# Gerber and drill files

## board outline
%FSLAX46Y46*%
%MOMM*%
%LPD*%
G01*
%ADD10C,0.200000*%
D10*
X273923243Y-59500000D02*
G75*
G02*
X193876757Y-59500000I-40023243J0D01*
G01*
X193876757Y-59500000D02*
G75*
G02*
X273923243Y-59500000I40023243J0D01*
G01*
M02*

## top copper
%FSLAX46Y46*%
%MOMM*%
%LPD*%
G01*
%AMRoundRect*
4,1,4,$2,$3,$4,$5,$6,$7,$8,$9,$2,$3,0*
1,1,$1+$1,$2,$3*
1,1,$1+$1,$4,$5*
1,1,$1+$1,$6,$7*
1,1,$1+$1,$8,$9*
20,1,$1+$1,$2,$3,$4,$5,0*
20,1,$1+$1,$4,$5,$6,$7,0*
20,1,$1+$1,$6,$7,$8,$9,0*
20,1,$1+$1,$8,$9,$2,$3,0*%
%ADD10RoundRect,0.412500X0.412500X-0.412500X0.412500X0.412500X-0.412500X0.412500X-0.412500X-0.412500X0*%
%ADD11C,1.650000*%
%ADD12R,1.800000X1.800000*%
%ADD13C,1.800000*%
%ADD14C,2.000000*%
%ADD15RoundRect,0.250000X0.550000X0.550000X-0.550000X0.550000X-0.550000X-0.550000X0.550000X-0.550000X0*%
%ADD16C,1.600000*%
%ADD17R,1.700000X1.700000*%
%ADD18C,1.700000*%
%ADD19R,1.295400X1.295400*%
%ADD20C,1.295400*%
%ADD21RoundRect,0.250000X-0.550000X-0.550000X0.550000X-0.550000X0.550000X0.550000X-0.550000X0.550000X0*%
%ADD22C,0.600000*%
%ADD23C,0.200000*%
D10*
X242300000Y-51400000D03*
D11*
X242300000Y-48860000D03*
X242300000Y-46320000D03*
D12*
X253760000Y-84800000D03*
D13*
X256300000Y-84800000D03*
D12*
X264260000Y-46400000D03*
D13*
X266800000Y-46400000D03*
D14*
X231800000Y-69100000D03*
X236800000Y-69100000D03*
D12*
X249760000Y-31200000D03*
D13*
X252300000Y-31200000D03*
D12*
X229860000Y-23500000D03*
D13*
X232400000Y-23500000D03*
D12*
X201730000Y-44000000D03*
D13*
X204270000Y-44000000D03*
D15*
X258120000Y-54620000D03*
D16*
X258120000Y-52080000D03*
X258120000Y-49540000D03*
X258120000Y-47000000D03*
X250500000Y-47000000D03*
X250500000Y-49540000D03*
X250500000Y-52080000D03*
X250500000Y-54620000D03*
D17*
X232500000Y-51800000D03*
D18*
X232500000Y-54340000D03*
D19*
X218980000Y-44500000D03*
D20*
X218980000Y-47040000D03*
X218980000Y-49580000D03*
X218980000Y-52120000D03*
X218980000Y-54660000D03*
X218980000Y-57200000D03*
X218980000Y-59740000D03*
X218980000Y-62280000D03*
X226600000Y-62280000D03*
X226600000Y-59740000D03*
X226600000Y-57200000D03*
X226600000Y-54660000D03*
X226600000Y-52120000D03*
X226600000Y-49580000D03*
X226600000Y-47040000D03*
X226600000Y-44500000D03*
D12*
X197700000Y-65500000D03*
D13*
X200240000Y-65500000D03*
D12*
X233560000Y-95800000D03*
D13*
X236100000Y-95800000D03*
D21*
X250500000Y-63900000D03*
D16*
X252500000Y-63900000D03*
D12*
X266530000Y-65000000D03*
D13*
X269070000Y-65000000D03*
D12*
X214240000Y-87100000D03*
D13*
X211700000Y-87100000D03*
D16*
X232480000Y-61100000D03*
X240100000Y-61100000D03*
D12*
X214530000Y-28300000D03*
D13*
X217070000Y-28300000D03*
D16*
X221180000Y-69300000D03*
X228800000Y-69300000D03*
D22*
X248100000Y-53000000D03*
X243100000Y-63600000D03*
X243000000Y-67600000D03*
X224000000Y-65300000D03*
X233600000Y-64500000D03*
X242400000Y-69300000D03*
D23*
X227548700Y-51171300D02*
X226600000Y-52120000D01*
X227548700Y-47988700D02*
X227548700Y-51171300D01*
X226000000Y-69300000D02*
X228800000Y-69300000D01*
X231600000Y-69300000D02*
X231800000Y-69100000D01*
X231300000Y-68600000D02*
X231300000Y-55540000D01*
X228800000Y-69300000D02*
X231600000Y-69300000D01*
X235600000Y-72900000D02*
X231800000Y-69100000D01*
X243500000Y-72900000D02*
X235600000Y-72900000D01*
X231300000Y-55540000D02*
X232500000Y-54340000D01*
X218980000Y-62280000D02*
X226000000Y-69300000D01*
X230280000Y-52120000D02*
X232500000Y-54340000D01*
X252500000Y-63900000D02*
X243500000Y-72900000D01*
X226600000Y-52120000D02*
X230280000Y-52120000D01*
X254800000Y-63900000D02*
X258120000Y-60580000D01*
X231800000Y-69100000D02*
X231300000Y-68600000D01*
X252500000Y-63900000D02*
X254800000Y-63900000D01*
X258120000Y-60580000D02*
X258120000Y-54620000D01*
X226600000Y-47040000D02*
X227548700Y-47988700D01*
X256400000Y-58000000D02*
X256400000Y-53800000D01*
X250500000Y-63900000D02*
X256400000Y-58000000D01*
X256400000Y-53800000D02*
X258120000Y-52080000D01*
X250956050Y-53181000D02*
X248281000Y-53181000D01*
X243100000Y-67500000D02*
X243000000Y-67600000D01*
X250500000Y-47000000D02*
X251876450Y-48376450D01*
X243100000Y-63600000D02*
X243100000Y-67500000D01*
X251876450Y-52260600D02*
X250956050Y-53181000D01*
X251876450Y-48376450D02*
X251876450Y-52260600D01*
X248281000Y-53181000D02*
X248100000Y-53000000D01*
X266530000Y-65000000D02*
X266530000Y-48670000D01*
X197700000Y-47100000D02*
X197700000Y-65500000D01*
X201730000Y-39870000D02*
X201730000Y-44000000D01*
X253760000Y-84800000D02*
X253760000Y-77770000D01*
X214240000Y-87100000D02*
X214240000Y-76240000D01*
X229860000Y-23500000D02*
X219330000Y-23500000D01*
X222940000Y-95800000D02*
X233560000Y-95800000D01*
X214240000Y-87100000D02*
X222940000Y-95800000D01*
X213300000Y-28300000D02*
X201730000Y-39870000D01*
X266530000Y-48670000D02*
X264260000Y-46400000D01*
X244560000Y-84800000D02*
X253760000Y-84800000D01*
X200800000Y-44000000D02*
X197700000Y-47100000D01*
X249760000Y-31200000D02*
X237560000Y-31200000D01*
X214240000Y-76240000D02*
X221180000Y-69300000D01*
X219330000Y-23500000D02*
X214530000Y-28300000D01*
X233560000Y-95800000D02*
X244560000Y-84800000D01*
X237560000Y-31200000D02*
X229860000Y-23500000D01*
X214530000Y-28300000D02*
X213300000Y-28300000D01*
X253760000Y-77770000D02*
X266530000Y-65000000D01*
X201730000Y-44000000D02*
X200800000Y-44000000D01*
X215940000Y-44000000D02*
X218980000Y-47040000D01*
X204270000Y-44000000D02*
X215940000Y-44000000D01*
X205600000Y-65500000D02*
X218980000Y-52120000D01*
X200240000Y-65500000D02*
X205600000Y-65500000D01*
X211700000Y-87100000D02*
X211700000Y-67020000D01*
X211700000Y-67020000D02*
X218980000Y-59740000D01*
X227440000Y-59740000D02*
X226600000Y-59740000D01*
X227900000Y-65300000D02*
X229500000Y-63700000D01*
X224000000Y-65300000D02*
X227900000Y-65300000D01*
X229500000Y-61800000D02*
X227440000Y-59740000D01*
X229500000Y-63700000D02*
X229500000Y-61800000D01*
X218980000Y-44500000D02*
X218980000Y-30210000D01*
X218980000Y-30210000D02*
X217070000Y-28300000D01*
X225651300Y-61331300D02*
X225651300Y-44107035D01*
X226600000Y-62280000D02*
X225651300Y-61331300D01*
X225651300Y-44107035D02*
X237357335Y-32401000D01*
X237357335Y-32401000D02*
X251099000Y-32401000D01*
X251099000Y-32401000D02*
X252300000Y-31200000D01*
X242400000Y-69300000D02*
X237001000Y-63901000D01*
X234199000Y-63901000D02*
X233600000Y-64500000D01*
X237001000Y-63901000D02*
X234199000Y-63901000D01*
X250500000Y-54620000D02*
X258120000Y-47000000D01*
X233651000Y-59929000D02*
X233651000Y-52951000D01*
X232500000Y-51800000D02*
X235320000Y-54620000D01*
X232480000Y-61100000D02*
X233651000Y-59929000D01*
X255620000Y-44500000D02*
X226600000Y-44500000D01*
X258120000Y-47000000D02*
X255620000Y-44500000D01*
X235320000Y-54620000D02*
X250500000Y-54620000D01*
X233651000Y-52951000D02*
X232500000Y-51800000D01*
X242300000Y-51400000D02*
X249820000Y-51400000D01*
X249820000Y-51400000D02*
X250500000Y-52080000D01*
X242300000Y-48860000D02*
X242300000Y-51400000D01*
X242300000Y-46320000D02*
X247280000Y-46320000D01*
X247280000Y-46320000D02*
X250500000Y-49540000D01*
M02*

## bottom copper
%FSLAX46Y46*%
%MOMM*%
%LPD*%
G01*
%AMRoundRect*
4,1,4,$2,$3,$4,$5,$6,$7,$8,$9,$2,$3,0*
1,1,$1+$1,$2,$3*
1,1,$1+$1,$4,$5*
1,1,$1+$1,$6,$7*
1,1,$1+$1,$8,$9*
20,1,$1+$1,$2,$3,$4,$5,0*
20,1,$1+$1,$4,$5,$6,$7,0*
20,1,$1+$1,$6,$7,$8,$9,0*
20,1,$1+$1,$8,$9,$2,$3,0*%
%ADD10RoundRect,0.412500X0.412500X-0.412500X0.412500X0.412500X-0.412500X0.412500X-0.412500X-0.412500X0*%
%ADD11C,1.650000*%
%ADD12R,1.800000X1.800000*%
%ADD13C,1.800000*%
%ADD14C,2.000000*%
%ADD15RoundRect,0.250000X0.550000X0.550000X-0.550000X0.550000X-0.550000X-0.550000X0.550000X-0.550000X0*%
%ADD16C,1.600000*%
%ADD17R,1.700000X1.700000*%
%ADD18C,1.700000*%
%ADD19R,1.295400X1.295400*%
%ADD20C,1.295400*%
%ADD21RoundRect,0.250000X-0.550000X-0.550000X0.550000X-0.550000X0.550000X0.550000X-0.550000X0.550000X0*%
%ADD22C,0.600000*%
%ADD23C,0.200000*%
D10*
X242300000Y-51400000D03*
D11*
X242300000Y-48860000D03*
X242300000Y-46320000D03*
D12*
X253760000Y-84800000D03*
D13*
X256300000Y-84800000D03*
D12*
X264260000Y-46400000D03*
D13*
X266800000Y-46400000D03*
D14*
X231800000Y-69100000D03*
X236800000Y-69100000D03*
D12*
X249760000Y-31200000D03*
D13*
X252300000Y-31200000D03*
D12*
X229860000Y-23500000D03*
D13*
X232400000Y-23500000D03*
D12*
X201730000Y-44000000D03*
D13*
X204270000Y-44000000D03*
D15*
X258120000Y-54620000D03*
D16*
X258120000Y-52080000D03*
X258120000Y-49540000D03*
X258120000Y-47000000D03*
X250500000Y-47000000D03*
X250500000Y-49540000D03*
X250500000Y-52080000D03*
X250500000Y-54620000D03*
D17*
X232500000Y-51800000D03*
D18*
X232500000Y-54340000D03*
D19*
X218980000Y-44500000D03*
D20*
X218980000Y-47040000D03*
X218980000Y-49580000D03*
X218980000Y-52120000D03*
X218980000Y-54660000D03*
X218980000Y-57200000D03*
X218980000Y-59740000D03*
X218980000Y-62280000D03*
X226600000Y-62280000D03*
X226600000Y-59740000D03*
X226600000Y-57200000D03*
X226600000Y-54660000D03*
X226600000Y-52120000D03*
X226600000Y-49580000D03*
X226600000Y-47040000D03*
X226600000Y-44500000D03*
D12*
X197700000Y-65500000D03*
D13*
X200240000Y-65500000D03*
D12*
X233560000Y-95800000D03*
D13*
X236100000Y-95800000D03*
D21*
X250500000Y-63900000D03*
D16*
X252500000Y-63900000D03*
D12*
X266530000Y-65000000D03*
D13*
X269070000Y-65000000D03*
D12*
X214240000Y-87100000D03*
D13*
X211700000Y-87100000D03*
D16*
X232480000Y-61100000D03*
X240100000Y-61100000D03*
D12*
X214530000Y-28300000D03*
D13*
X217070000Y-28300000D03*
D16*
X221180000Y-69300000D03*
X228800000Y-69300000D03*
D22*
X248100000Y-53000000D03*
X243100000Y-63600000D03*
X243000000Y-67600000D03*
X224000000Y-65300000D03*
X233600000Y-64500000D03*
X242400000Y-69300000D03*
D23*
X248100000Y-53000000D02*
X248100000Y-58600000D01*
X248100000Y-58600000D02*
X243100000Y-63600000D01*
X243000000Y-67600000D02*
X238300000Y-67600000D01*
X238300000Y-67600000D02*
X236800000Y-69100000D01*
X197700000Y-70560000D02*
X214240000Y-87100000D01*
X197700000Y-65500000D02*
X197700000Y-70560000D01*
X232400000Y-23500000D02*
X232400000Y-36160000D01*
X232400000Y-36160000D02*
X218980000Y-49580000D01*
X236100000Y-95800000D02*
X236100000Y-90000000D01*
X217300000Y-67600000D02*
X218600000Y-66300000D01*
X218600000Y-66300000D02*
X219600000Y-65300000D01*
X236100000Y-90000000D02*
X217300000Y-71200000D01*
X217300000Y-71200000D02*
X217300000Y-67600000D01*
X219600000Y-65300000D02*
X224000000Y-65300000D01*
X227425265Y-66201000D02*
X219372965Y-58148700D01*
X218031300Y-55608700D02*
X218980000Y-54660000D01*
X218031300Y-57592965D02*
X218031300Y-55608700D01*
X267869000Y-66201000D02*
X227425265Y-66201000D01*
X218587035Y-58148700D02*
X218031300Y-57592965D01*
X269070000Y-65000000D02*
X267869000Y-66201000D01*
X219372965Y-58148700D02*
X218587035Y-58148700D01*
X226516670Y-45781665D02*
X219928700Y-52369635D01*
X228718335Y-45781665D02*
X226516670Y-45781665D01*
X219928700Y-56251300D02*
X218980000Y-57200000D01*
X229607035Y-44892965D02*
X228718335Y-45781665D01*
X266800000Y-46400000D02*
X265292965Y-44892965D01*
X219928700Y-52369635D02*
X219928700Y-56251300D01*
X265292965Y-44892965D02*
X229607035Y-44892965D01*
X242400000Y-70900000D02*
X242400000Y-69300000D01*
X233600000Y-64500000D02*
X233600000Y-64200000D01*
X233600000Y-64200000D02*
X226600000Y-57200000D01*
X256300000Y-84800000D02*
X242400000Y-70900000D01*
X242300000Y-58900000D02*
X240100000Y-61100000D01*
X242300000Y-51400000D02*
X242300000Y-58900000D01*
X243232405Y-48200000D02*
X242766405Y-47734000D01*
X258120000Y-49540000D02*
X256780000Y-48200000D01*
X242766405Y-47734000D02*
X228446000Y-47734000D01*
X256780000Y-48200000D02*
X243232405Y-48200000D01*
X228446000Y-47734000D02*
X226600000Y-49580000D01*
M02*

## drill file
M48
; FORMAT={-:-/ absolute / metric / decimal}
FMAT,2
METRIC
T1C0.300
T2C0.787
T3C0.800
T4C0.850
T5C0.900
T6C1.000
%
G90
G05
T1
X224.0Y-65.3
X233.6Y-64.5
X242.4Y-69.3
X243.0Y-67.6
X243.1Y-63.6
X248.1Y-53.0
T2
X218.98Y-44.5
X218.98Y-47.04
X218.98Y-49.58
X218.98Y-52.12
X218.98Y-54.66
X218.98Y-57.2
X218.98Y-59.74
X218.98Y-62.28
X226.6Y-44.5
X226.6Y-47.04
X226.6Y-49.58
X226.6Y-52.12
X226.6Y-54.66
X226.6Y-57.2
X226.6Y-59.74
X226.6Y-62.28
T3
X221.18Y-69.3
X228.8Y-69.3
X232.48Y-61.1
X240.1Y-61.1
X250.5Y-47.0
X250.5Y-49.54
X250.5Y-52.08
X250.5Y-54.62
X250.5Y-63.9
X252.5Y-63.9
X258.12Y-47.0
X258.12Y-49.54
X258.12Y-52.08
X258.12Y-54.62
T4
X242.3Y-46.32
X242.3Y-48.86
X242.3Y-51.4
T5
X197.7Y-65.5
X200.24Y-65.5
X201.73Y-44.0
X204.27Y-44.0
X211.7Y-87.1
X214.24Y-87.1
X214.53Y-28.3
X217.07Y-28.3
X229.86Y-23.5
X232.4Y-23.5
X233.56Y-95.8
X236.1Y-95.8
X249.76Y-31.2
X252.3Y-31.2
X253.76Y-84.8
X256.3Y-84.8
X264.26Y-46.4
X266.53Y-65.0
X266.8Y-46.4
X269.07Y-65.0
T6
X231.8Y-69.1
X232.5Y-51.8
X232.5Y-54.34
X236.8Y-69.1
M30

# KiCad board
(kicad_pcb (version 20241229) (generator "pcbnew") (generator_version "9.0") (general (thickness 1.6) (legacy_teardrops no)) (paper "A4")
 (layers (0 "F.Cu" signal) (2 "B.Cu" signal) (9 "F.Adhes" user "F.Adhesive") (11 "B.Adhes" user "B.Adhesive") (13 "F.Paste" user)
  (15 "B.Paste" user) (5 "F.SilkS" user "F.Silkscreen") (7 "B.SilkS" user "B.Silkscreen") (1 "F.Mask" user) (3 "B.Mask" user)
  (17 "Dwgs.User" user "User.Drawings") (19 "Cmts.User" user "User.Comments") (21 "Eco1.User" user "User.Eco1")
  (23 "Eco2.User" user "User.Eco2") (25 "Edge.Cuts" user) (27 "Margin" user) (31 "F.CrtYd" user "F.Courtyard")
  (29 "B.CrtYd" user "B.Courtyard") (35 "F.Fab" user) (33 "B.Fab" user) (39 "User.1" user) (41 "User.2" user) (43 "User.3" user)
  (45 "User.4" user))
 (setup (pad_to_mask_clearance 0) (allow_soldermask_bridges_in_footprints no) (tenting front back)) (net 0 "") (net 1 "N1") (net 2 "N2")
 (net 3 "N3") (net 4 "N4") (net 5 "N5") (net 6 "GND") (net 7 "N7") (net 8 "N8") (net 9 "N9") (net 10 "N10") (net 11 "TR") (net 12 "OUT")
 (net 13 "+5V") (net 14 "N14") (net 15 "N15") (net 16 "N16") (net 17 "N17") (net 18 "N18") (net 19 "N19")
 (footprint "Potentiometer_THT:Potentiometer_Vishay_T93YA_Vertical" (layer "F.Cu") (at 242.3 51.4 90)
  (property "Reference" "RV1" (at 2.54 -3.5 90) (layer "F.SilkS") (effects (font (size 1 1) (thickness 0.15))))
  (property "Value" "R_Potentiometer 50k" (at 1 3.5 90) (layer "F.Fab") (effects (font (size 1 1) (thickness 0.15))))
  (pad "1" thru_hole roundrect (at 0 0 90) (size 1.65 1.65) (drill 0.85) (layers "*.Cu" "*.Mask") (remove_unused_layers no)
   (roundrect_rratio 0.25) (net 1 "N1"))
  (pad "2" thru_hole circle (at 2.54 0 90) (size 1.65 1.65) (drill 0.85) (layers "*.Cu" "*.Mask") (remove_unused_layers no) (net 1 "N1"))
  (pad "3" thru_hole circle (at 5.08 0 90) (size 1.65 1.65) (drill 0.85) (layers "*.Cu" "*.Mask") (remove_unused_layers no) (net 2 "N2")))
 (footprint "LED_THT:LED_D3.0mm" (layer "F.Cu") (at 253.76 84.8)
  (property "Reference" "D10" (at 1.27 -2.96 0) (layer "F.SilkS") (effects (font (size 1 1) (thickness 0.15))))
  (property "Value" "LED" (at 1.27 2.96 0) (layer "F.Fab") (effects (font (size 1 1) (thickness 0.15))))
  (pad "1" thru_hole rect (at 0 0) (size 1.8 1.8) (drill 0.9) (layers "*.Cu" "*.Mask") (remove_unused_layers no) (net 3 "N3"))
  (pad "2" thru_hole circle (at 2.54 0) (size 1.8 1.8) (drill 0.9) (layers "*.Cu" "*.Mask") (remove_unused_layers no) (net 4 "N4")))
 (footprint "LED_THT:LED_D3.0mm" (layer "F.Cu") (at 264.26 46.4)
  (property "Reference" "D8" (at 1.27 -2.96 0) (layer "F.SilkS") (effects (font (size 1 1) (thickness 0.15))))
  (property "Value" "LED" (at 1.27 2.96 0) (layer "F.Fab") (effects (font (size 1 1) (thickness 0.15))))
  (pad "1" thru_hole rect (at 0 0) (size 1.8 1.8) (drill 0.9) (layers "*.Cu" "*.Mask") (remove_unused_layers no) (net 3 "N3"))
  (pad "2" thru_hole circle (at 2.54 0) (size 1.8 1.8) (drill 0.9) (layers "*.Cu" "*.Mask") (remove_unused_layers no) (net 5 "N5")))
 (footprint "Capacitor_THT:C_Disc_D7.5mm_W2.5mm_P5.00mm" (layer "F.Cu") (at 231.8 69.1)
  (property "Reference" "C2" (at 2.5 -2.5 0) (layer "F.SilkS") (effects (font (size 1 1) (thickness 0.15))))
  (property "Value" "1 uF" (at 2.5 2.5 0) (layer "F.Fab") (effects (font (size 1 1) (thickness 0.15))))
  (pad "1" thru_hole circle (at 0 0) (size 2 2) (drill 1) (layers "*.Cu" "*.Mask") (remove_unused_layers no) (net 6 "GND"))
  (pad "2" thru_hole circle (at 5 0) (size 2 2) (drill 1) (layers "*.Cu" "*.Mask") (remove_unused_layers no) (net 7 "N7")))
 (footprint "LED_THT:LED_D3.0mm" (layer "F.Cu") (at 249.76 31.2)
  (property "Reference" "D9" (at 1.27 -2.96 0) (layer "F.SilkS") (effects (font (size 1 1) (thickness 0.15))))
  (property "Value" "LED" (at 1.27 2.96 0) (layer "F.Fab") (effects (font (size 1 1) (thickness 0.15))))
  (pad "1" thru_hole rect (at 0 0) (size 1.8 1.8) (drill 0.9) (layers "*.Cu" "*.Mask") (remove_unused_layers no) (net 3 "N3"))
  (pad "2" thru_hole circle (at 2.54 0) (size 1.8 1.8) (drill 0.9) (layers "*.Cu" "*.Mask") (remove_unused_layers no) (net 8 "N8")))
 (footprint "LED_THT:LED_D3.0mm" (layer "F.Cu") (at 229.86 23.5)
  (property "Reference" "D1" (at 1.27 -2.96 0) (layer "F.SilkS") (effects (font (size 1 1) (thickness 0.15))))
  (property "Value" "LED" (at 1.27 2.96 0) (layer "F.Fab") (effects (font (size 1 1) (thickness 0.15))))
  (pad "1" thru_hole rect (at 0 0) (size 1.8 1.8) (drill 0.9) (layers "*.Cu" "*.Mask") (remove_unused_layers no) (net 3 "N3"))
  (pad "2" thru_hole circle (at 2.54 0) (size 1.8 1.8) (drill 0.9) (layers "*.Cu" "*.Mask") (remove_unused_layers no) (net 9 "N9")))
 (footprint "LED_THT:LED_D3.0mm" (layer "F.Cu") (at 201.73 44)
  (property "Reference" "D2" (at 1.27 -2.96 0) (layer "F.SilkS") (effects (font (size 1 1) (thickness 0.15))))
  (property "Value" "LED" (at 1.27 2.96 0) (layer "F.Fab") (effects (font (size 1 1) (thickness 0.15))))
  (pad "1" thru_hole rect (at 0 0) (size 1.8 1.8) (drill 0.9) (layers "*.Cu" "*.Mask") (remove_unused_layers no) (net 3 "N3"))
  (pad "2" thru_hole circle (at 2.54 0) (size 1.8 1.8) (drill 0.9) (layers "*.Cu" "*.Mask") (remove_unused_layers no) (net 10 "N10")))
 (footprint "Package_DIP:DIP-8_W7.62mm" (layer "F.Cu") (at 258.12 54.62 180)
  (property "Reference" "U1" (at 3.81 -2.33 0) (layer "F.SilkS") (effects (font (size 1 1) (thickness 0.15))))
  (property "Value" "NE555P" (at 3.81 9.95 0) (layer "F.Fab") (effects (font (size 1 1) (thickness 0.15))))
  (pad "1" thru_hole roundrect (at 0 0 180) (size 1.6 1.6) (drill 0.8) (layers "*.Cu" "*.Mask") (remove_unused_layers no)
   (roundrect_rratio 0.15625) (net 6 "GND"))
  (pad "2" thru_hole circle (at 0 2.54 180) (size 1.6 1.6) (drill 0.8) (layers "*.Cu" "*.Mask") (remove_unused_layers no) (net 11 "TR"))
  (pad "3" thru_hole circle (at 0 5.08 180) (size 1.6 1.6) (drill 0.8) (layers "*.Cu" "*.Mask") (remove_unused_layers no) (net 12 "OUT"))
  (pad "4" thru_hole circle (at 0 7.62 180) (size 1.6 1.6) (drill 0.8) (layers "*.Cu" "*.Mask") (remove_unused_layers no) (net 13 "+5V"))
  (pad "5" thru_hole circle (at 7.62 7.62 180) (size 1.6 1.6) (drill 0.8) (layers "*.Cu" "*.Mask") (remove_unused_layers no) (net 7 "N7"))
  (pad "6" thru_hole circle (at 7.62 5.08 180) (size 1.6 1.6) (drill 0.8) (layers "*.Cu" "*.Mask") (remove_unused_layers no) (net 2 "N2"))
  (pad "7" thru_hole circle (at 7.62 2.54 180) (size 1.6 1.6) (drill 0.8) (layers "*.Cu" "*.Mask") (remove_unused_layers no) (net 1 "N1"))
  (pad "8" thru_hole circle (at 7.62 0 180) (size 1.6 1.6) (drill 0.8) (layers "*.Cu" "*.Mask") (remove_unused_layers no) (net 13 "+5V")))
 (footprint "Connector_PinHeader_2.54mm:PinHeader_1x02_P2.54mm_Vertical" (layer "F.Cu") (at 232.5 51.8)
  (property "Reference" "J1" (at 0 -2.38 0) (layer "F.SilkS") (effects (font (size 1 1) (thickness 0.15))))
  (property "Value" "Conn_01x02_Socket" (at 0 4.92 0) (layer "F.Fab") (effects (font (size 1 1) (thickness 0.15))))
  (pad "1" thru_hole rect (at 0 0) (size 1.7 1.7) (drill 1) (layers "*.Cu" "*.Mask") (remove_unused_layers no) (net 13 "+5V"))
  (pad "2" thru_hole circle (at 0 2.54) (size 1.7 1.7) (drill 1) (layers "*.Cu" "*.Mask") (remove_unused_layers no) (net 6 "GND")))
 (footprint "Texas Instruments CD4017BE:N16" (layer "F.Cu") (at 226.6 62.28)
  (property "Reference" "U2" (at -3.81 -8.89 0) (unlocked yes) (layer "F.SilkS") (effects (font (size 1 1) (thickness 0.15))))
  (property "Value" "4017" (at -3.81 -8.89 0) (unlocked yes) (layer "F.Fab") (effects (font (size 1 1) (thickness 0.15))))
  (pad "1" thru_hole rect (at -7.62 -17.78) (size 1.2954 1.2954) (drill 0.7874) (layers "*.Cu" "*.Mask") (remove_unused_layers no)
   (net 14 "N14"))
  (pad "2" thru_hole circle (at -7.62 -15.24) (size 1.2954 1.2954) (drill 0.7874) (layers "*.Cu" "*.Mask") (remove_unused_layers no)
   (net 10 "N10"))
  (pad "3" thru_hole circle (at -7.62 -12.7) (size 1.2954 1.2954) (drill 0.7874) (layers "*.Cu" "*.Mask") (remove_unused_layers no)
   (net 9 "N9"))
  (pad "4" thru_hole circle (at -7.62 -10.16) (size 1.2954 1.2954) (drill 0.7874) (layers "*.Cu" "*.Mask") (remove_unused_layers no)
   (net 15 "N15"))
  (pad "5" thru_hole circle (at -7.62 -7.62) (size 1.2954 1.2954) (drill 0.7874) (layers "*.Cu" "*.Mask") (remove_unused_layers no)
   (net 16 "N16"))
  (pad "6" thru_hole circle (at -7.62 -5.08) (size 1.2954 1.2954) (drill 0.7874) (layers "*.Cu" "*.Mask") (remove_unused_layers no)
   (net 5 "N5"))
  (pad "7" thru_hole circle (at -7.62 -2.54) (size 1.2954 1.2954) (drill 0.7874) (layers "*.Cu" "*.Mask") (remove_unused_layers no)
   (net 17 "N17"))
  (pad "8" thru_hole circle (at -7.62 0) (size 1.2954 1.2954) (drill 0.7874) (layers "*.Cu" "*.Mask") (remove_unused_layers no)
   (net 6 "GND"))
  (pad "9" thru_hole circle (at 0 0) (size 1.2954 1.2954) (drill 0.7874) (layers "*.Cu" "*.Mask") (remove_unused_layers no) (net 8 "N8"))
  (pad "10" thru_hole circle (at 0 -2.54) (size 1.2954 1.2954) (drill 0.7874) (layers "*.Cu" "*.Mask") (remove_unused_layers no)
   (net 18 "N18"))
  (pad "11" thru_hole circle (at 0 -5.08) (size 1.2954 1.2954) (drill 0.7874) (layers "*.Cu" "*.Mask") (remove_unused_layers no)
   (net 4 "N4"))
  (pad "12" thru_hole circle (at 0 -7.62) (size 1.2954 1.2954) (drill 0.7874) (layers "*.Cu" "*.Mask") (remove_unused_layers no)
   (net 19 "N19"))
  (pad "13" thru_hole circle (at 0 -10.16) (size 1.2954 1.2954) (drill 0.7874) (layers "*.Cu" "*.Mask") (remove_unused_layers no)
   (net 6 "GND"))
  (pad "14" thru_hole circle (at 0 -12.7) (size 1.2954 1.2954) (drill 0.7874) (layers "*.Cu" "*.Mask") (remove_unused_layers no)
   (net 12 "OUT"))
  (pad "15" thru_hole circle (at 0 -15.24) (size 1.2954 1.2954) (drill 0.7874) (layers "*.Cu" "*.Mask") (remove_unused_layers no)
   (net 6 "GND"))
  (pad "16" thru_hole circle (at 0 -17.78) (size 1.2954 1.2954) (drill 0.7874) (layers "*.Cu" "*.Mask") (remove_unused_layers no)
   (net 13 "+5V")))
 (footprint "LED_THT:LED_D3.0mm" (layer "F.Cu") (at 197.7 65.5)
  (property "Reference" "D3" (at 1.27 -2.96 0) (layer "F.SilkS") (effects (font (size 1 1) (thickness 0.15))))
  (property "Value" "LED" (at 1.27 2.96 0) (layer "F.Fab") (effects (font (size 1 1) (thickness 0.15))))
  (pad "1" thru_hole rect (at 0 0) (size 1.8 1.8) (drill 0.9) (layers "*.Cu" "*.Mask") (remove_unused_layers no) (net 3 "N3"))
  (pad "2" thru_hole circle (at 2.54 0) (size 1.8 1.8) (drill 0.9) (layers "*.Cu" "*.Mask") (remove_unused_layers no) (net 15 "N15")))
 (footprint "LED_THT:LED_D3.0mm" (layer "F.Cu") (at 233.56 95.8)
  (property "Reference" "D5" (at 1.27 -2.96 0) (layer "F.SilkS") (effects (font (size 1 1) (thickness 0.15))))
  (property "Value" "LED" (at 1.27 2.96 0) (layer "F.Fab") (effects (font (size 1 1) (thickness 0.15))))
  (pad "1" thru_hole rect (at 0 0) (size 1.8 1.8) (drill 0.9) (layers "*.Cu" "*.Mask") (remove_unused_layers no) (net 3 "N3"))
  (pad "2" thru_hole circle (at 2.54 0) (size 1.8 1.8) (drill 0.9) (layers "*.Cu" "*.Mask") (remove_unused_layers no) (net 18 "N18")))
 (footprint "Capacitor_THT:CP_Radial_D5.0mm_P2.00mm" (layer "F.Cu") (at 250.5 63.9)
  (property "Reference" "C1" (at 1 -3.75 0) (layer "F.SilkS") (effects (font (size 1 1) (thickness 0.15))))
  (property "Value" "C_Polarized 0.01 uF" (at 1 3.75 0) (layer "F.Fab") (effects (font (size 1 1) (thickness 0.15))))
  (pad "1" thru_hole roundrect (at 0 0) (size 1.6 1.6) (drill 0.8) (layers "*.Cu" "*.Mask") (remove_unused_layers no)
   (roundrect_rratio 0.15625) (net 11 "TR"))
  (pad "2" thru_hole circle (at 2 0) (size 1.6 1.6) (drill 0.8) (layers "*.Cu" "*.Mask") (remove_unused_layers no) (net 6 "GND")))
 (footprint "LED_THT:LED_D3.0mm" (layer "F.Cu") (at 266.53 65)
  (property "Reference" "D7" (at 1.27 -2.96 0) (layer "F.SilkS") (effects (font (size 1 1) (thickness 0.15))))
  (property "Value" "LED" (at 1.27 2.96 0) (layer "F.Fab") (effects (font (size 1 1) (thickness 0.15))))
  (pad "1" thru_hole rect (at 0 0) (size 1.8 1.8) (drill 0.9) (layers "*.Cu" "*.Mask") (remove_unused_layers no) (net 3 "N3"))
  (pad "2" thru_hole circle (at 2.54 0) (size 1.8 1.8) (drill 0.9) (layers "*.Cu" "*.Mask") (remove_unused_layers no) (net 16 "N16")))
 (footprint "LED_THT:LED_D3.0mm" (layer "F.Cu") (at 214.24 87.1 180)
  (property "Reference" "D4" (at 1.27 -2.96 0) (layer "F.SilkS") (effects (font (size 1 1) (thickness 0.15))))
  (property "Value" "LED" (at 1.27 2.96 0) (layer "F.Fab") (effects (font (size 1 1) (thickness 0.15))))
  (pad "1" thru_hole rect (at 0 0 180) (size 1.8 1.8) (drill 0.9) (layers "*.Cu" "*.Mask") (remove_unused_layers no) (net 3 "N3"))
  (pad "2" thru_hole circle (at 2.54 0 180) (size 1.8 1.8) (drill 0.9) (layers "*.Cu" "*.Mask") (remove_unused_layers no) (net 17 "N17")))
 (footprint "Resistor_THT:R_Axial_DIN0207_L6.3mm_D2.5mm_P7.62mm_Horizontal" (layer "F.Cu") (at 232.48 61.1)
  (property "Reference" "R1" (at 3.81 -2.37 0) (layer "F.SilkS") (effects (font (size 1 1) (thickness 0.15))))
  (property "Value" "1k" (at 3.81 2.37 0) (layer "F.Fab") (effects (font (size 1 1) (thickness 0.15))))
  (pad "1" thru_hole circle (at 0 0) (size 1.6 1.6) (drill 0.8) (layers "*.Cu" "*.Mask") (remove_unused_layers no) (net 13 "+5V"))
  (pad "2" thru_hole circle (at 7.62 0) (size 1.6 1.6) (drill 0.8) (layers "*.Cu" "*.Mask") (remove_unused_layers no) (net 1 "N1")))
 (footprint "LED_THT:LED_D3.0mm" (layer "F.Cu") (at 214.53 28.3)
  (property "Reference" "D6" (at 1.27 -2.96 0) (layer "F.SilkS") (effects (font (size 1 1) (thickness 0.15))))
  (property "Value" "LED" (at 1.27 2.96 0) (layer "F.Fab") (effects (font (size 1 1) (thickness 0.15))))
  (pad "1" thru_hole rect (at 0 0) (size 1.8 1.8) (drill 0.9) (layers "*.Cu" "*.Mask") (remove_unused_layers no) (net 3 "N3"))
  (pad "2" thru_hole circle (at 2.54 0) (size 1.8 1.8) (drill 0.9) (layers "*.Cu" "*.Mask") (remove_unused_layers no) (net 14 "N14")))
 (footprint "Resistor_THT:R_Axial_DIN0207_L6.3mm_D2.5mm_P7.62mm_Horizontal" (layer "F.Cu") (at 221.18 69.3)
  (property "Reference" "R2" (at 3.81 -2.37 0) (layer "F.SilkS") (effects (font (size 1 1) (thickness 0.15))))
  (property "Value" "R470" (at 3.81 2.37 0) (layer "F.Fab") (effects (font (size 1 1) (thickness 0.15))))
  (pad "1" thru_hole circle (at 0 0) (size 1.6 1.6) (drill 0.8) (layers "*.Cu" "*.Mask") (remove_unused_layers no) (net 3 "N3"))
  (pad "2" thru_hole circle (at 7.62 0) (size 1.6 1.6) (drill 0.8) (layers "*.Cu" "*.Mask") (remove_unused_layers no) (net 6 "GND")))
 (gr_circle (center 233.9 59.5) (end 267 82) (stroke (width 0.2) (type solid)) (fill no) (layer "Edge.Cuts"))
 (segment (start 227.5487 51.1713) (end 226.6 52.12) (width 0.2) (layer "F.Cu") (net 6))
 (segment (start 227.5487 47.9887) (end 227.5487 51.1713) (width 0.2) (layer "F.Cu") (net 6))
 (segment (start 226 69.3) (end 228.8 69.3) (width 0.2) (layer "F.Cu") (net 6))
 (segment (start 231.6 69.3) (end 231.8 69.1) (width 0.2) (layer "F.Cu") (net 6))
 (segment (start 231.3 68.6) (end 231.3 55.54) (width 0.2) (layer "F.Cu") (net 6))
 (segment (start 228.8 69.3) (end 231.6 69.3) (width 0.2) (layer "F.Cu") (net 6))
 (segment (start 235.6 72.9) (end 231.8 69.1) (width 0.2) (layer "F.Cu") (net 6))
 (segment (start 243.5 72.9) (end 235.6 72.9) (width 0.2) (layer "F.Cu") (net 6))
 (segment (start 231.3 55.54) (end 232.5 54.34) (width 0.2) (layer "F.Cu") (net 6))
 (segment (start 218.98 62.28) (end 226 69.3) (width 0.2) (layer "F.Cu") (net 6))
 (segment (start 230.28 52.12) (end 232.5 54.34) (width 0.2) (layer "F.Cu") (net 6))
 (segment (start 252.5 63.9) (end 243.5 72.9) (width 0.2) (layer "F.Cu") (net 6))
 (segment (start 226.6 52.12) (end 230.28 52.12) (width 0.2) (layer "F.Cu") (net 6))
 (segment (start 254.8 63.9) (end 258.12 60.58) (width 0.2) (layer "F.Cu") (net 6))
 (segment (start 231.8 69.1) (end 231.3 68.6) (width 0.2) (layer "F.Cu") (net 6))
 (segment (start 252.5 63.9) (end 254.8 63.9) (width 0.2) (layer "F.Cu") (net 6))
 (segment (start 258.12 60.58) (end 258.12 54.62) (width 0.2) (layer "F.Cu") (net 6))
 (segment (start 226.6 47.04) (end 227.5487 47.9887) (width 0.2) (layer "F.Cu") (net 6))
 (segment (start 256.4 58) (end 256.4 53.8) (width 0.2) (layer "F.Cu") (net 11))
 (segment (start 250.5 63.9) (end 256.4 58) (width 0.2) (layer "F.Cu") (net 11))
 (segment (start 256.4 53.8) (end 258.12 52.08) (width 0.2) (layer "F.Cu") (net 11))
 (segment (start 250.95605 53.181) (end 248.281 53.181) (width 0.2) (layer "F.Cu") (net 7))
 (segment (start 243.1 67.5) (end 243 67.6) (width 0.2) (layer "F.Cu") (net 7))
 (segment (start 250.5 47) (end 251.87645 48.37645) (width 0.2) (layer "F.Cu") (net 7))
 (segment (start 243.1 63.6) (end 243.1 67.5) (width 0.2) (layer "F.Cu") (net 7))
 (segment (start 251.87645 52.2606) (end 250.95605 53.181) (width 0.2) (layer "F.Cu") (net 7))
 (segment (start 251.87645 48.37645) (end 251.87645 52.2606) (width 0.2) (layer "F.Cu") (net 7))
 (segment (start 248.281 53.181) (end 248.1 53) (width 0.2) (layer "F.Cu") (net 7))
 (via (at 248.1 53) (size 0.6) (drill 0.3) (layers "F.Cu" "B.Cu") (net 7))
 (via (at 243.1 63.6) (size 0.6) (drill 0.3) (layers "F.Cu" "B.Cu") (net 7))
 (via (at 243 67.6) (size 0.6) (drill 0.3) (layers "F.Cu" "B.Cu") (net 7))
 (segment (start 248.1 53) (end 248.1 58.6) (width 0.2) (layer "B.Cu") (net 7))
 (segment (start 248.1 58.6) (end 243.1 63.6) (width 0.2) (layer "B.Cu") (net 7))
 (segment (start 243 67.6) (end 238.3 67.6) (width 0.2) (layer "B.Cu") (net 7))
 (segment (start 238.3 67.6) (end 236.8 69.1) (width 0.2) (layer "B.Cu") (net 7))
 (segment (start 266.53 65) (end 266.53 48.67) (width 0.2) (layer "F.Cu") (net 3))
 (segment (start 197.7 47.1) (end 197.7 65.5) (width 0.2) (layer "F.Cu") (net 3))
 (segment (start 201.73 39.87) (end 201.73 44) (width 0.2) (layer "F.Cu") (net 3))
 (segment (start 253.76 84.8) (end 253.76 77.77) (width 0.2) (layer "F.Cu") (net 3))
 (segment (start 214.24 87.1) (end 214.24 76.24) (width 0.2) (layer "F.Cu") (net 3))
 (segment (start 229.86 23.5) (end 219.33 23.5) (width 0.2) (layer "F.Cu") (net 3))
 (segment (start 222.94 95.8) (end 233.56 95.8) (width 0.2) (layer "F.Cu") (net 3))
 (segment (start 214.24 87.1) (end 222.94 95.8) (width 0.2) (layer "F.Cu") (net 3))
 (segment (start 213.3 28.3) (end 201.73 39.87) (width 0.2) (layer "F.Cu") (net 3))
 (segment (start 266.53 48.67) (end 264.26 46.4) (width 0.2) (layer "F.Cu") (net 3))
 (segment (start 244.56 84.8) (end 253.76 84.8) (width 0.2) (layer "F.Cu") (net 3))
 (segment (start 200.8 44) (end 197.7 47.1) (width 0.2) (layer "F.Cu") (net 3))
 (segment (start 249.76 31.2) (end 237.56 31.2) (width 0.2) (layer "F.Cu") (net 3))
 (segment (start 214.24 76.24) (end 221.18 69.3) (width 0.2) (layer "F.Cu") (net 3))
 (segment (start 219.33 23.5) (end 214.53 28.3) (width 0.2) (layer "F.Cu") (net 3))
 (segment (start 233.56 95.8) (end 244.56 84.8) (width 0.2) (layer "F.Cu") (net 3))
 (segment (start 237.56 31.2) (end 229.86 23.5) (width 0.2) (layer "F.Cu") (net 3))
 (segment (start 214.53 28.3) (end 213.3 28.3) (width 0.2) (layer "F.Cu") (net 3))
 (segment (start 253.76 77.77) (end 266.53 65) (width 0.2) (layer "F.Cu") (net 3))
 (segment (start 201.73 44) (end 200.8 44) (width 0.2) (layer "F.Cu") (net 3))
 (segment (start 197.7 70.56) (end 214.24 87.1) (width 0.2) (layer "B.Cu") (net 3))
 (segment (start 197.7 65.5) (end 197.7 70.56) (width 0.2) (layer "B.Cu") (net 3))
 (segment (start 232.4 23.5) (end 232.4 36.16) (width 0.2) (layer "B.Cu") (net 9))
 (segment (start 232.4 36.16) (end 218.98 49.58) (width 0.2) (layer "B.Cu") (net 9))
 (segment (start 215.94 44) (end 218.98 47.04) (width 0.2) (layer "F.Cu") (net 10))
 (segment (start 204.27 44) (end 215.94 44) (width 0.2) (layer "F.Cu") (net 10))
 (segment (start 205.6 65.5) (end 218.98 52.12) (width 0.2) (layer "F.Cu") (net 15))
 (segment (start 200.24 65.5) (end 205.6 65.5) (width 0.2) (layer "F.Cu") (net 15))
 (segment (start 211.7 87.1) (end 211.7 67.02) (width 0.2) (layer "F.Cu") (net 17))
 (segment (start 211.7 67.02) (end 218.98 59.74) (width 0.2) (layer "F.Cu") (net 17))
 (segment (start 227.44 59.74) (end 226.6 59.74) (width 0.2) (layer "F.Cu") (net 18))
 (segment (start 227.9 65.3) (end 229.5 63.7) (width 0.2) (layer "F.Cu") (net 18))
 (segment (start 224 65.3) (end 227.9 65.3) (width 0.2) (layer "F.Cu") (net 18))
 (segment (start 229.5 61.8) (end 227.44 59.74) (width 0.2) (layer "F.Cu") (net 18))
 (segment (start 229.5 63.7) (end 229.5 61.8) (width 0.2) (layer "F.Cu") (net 18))
 (via (at 224 65.3) (size 0.6) (drill 0.3) (layers "F.Cu" "B.Cu") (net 18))
 (segment (start 236.1 95.8) (end 236.1 90) (width 0.2) (layer "B.Cu") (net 18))
 (segment (start 217.3 67.6) (end 218.6 66.3) (width 0.2) (layer "B.Cu") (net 18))
 (segment (start 218.6 66.3) (end 219.6 65.3) (width 0.2) (layer "B.Cu") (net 18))
 (segment (start 236.1 90) (end 217.3 71.2) (width 0.2) (layer "B.Cu") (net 18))
 (segment (start 217.3 71.2) (end 217.3 67.6) (width 0.2) (layer "B.Cu") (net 18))
 (segment (start 219.6 65.3) (end 224 65.3) (width 0.2) (layer "B.Cu") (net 18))
 (segment (start 218.98 44.5) (end 218.98 30.21) (width 0.2) (layer "F.Cu") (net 14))
 (segment (start 218.98 30.21) (end 217.07 28.3) (width 0.2) (layer "F.Cu") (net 14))
 (segment (start 227.425265 66.201) (end 219.372965 58.1487) (width 0.2) (layer "B.Cu") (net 16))
 (segment (start 218.0313 55.6087) (end 218.98 54.66) (width 0.2) (layer "B.Cu") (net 16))
 (segment (start 218.0313 57.592965) (end 218.0313 55.6087) (width 0.2) (layer "B.Cu") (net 16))
 (segment (start 267.869 66.201) (end 227.425265 66.201) (width 0.2) (layer "B.Cu") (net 16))
 (segment (start 218.587035 58.1487) (end 218.0313 57.592965) (width 0.2) (layer "B.Cu") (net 16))
 (segment (start 269.07 65) (end 267.869 66.201) (width 0.2) (layer "B.Cu") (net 16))
 (segment (start 219.372965 58.1487) (end 218.587035 58.1487) (width 0.2) (layer "B.Cu") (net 16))
 (segment (start 226.51667 45.781665) (end 219.9287 52.369635) (width 0.2) (layer "B.Cu") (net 5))
 (segment (start 228.718335 45.781665) (end 226.51667 45.781665) (width 0.2) (layer "B.Cu") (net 5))
 (segment (start 219.9287 56.2513) (end 218.98 57.2) (width 0.2) (layer "B.Cu") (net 5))
 (segment (start 229.607035 44.892965) (end 228.718335 45.781665) (width 0.2) (layer "B.Cu") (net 5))
 (segment (start 266.8 46.4) (end 265.292965 44.892965) (width 0.2) (layer "B.Cu") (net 5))
 (segment (start 219.9287 52.369635) (end 219.9287 56.2513) (width 0.2) (layer "B.Cu") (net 5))
 (segment (start 265.292965 44.892965) (end 229.607035 44.892965) (width 0.2) (layer "B.Cu") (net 5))
 (segment (start 225.6513 61.3313) (end 225.6513 44.107035) (width 0.2) (layer "F.Cu") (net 8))
 (segment (start 226.6 62.28) (end 225.6513 61.3313) (width 0.2) (layer "F.Cu") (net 8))
 (segment (start 225.6513 44.107035) (end 237.357335 32.401) (width 0.2) (layer "F.Cu") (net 8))
 (segment (start 237.357335 32.401) (end 251.099 32.401) (width 0.2) (layer "F.Cu") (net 8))
 (segment (start 251.099 32.401) (end 252.3 31.2) (width 0.2) (layer "F.Cu") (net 8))
 (segment (start 242.4 69.3) (end 237.001 63.901) (width 0.2) (layer "F.Cu") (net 4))
 (segment (start 234.199 63.901) (end 233.6 64.5) (width 0.2) (layer "F.Cu") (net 4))
 (segment (start 237.001 63.901) (end 234.199 63.901) (width 0.2) (layer "F.Cu") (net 4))
 (via (at 233.6 64.5) (size 0.6) (drill 0.3) (layers "F.Cu" "B.Cu") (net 4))
 (via (at 242.4 69.3) (size 0.6) (drill 0.3) (layers "F.Cu" "B.Cu") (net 4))
 (segment (start 242.4 70.9) (end 242.4 69.3) (width 0.2) (layer "B.Cu") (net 4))
 (segment (start 233.6 64.5) (end 233.6 64.2) (width 0.2) (layer "B.Cu") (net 4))
 (segment (start 233.6 64.2) (end 226.6 57.2) (width 0.2) (layer "B.Cu") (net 4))
 (segment (start 256.3 84.8) (end 242.4 70.9) (width 0.2) (layer "B.Cu") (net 4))
 (segment (start 250.5 54.62) (end 258.12 47) (width 0.2) (layer "F.Cu") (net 13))
 (segment (start 233.651 59.929) (end 233.651 52.951) (width 0.2) (layer "F.Cu") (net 13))
 (segment (start 232.5 51.8) (end 235.32 54.62) (width 0.2) (layer "F.Cu") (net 13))
 (segment (start 232.48 61.1) (end 233.651 59.929) (width 0.2) (layer "F.Cu") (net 13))
 (segment (start 255.62 44.5) (end 226.6 44.5) (width 0.2) (layer "F.Cu") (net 13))
 (segment (start 258.12 47) (end 255.62 44.5) (width 0.2) (layer "F.Cu") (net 13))
 (segment (start 235.32 54.62) (end 250.5 54.62) (width 0.2) (layer "F.Cu") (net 13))
 (segment (start 233.651 52.951) (end 232.5 51.8) (width 0.2) (layer "F.Cu") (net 13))
 (segment (start 242.3 51.4) (end 249.82 51.4) (width 0.2) (layer "F.Cu") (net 1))
 (segment (start 249.82 51.4) (end 250.5 52.08) (width 0.2) (layer "F.Cu") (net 1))
 (segment (start 242.3 48.86) (end 242.3 51.4) (width 0.2) (layer "F.Cu") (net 1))
 (segment (start 242.3 58.9) (end 240.1 61.1) (width 0.2) (layer "B.Cu") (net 1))
 (segment (start 242.3 51.4) (end 242.3 58.9) (width 0.2) (layer "B.Cu") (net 1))
 (segment (start 242.3 46.32) (end 247.28 46.32) (width 0.2) (layer "F.Cu") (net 2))
 (segment (start 247.28 46.32) (end 250.5 49.54) (width 0.2) (layer "F.Cu") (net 2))
 (segment (start 243.232405 48.2) (end 242.766405 47.734) (width 0.2) (layer "B.Cu") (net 12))
 (segment (start 258.12 49.54) (end 256.78 48.2) (width 0.2) (layer "B.Cu") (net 12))
 (segment (start 242.766405 47.734) (end 228.446 47.734) (width 0.2) (layer "B.Cu") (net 12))
 (segment (start 256.78 48.2) (end 243.232405 48.2) (width 0.2) (layer "B.Cu") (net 12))
 (segment (start 228.446 47.734) (end 226.6 49.58) (width 0.2) (layer "B.Cu") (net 12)))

